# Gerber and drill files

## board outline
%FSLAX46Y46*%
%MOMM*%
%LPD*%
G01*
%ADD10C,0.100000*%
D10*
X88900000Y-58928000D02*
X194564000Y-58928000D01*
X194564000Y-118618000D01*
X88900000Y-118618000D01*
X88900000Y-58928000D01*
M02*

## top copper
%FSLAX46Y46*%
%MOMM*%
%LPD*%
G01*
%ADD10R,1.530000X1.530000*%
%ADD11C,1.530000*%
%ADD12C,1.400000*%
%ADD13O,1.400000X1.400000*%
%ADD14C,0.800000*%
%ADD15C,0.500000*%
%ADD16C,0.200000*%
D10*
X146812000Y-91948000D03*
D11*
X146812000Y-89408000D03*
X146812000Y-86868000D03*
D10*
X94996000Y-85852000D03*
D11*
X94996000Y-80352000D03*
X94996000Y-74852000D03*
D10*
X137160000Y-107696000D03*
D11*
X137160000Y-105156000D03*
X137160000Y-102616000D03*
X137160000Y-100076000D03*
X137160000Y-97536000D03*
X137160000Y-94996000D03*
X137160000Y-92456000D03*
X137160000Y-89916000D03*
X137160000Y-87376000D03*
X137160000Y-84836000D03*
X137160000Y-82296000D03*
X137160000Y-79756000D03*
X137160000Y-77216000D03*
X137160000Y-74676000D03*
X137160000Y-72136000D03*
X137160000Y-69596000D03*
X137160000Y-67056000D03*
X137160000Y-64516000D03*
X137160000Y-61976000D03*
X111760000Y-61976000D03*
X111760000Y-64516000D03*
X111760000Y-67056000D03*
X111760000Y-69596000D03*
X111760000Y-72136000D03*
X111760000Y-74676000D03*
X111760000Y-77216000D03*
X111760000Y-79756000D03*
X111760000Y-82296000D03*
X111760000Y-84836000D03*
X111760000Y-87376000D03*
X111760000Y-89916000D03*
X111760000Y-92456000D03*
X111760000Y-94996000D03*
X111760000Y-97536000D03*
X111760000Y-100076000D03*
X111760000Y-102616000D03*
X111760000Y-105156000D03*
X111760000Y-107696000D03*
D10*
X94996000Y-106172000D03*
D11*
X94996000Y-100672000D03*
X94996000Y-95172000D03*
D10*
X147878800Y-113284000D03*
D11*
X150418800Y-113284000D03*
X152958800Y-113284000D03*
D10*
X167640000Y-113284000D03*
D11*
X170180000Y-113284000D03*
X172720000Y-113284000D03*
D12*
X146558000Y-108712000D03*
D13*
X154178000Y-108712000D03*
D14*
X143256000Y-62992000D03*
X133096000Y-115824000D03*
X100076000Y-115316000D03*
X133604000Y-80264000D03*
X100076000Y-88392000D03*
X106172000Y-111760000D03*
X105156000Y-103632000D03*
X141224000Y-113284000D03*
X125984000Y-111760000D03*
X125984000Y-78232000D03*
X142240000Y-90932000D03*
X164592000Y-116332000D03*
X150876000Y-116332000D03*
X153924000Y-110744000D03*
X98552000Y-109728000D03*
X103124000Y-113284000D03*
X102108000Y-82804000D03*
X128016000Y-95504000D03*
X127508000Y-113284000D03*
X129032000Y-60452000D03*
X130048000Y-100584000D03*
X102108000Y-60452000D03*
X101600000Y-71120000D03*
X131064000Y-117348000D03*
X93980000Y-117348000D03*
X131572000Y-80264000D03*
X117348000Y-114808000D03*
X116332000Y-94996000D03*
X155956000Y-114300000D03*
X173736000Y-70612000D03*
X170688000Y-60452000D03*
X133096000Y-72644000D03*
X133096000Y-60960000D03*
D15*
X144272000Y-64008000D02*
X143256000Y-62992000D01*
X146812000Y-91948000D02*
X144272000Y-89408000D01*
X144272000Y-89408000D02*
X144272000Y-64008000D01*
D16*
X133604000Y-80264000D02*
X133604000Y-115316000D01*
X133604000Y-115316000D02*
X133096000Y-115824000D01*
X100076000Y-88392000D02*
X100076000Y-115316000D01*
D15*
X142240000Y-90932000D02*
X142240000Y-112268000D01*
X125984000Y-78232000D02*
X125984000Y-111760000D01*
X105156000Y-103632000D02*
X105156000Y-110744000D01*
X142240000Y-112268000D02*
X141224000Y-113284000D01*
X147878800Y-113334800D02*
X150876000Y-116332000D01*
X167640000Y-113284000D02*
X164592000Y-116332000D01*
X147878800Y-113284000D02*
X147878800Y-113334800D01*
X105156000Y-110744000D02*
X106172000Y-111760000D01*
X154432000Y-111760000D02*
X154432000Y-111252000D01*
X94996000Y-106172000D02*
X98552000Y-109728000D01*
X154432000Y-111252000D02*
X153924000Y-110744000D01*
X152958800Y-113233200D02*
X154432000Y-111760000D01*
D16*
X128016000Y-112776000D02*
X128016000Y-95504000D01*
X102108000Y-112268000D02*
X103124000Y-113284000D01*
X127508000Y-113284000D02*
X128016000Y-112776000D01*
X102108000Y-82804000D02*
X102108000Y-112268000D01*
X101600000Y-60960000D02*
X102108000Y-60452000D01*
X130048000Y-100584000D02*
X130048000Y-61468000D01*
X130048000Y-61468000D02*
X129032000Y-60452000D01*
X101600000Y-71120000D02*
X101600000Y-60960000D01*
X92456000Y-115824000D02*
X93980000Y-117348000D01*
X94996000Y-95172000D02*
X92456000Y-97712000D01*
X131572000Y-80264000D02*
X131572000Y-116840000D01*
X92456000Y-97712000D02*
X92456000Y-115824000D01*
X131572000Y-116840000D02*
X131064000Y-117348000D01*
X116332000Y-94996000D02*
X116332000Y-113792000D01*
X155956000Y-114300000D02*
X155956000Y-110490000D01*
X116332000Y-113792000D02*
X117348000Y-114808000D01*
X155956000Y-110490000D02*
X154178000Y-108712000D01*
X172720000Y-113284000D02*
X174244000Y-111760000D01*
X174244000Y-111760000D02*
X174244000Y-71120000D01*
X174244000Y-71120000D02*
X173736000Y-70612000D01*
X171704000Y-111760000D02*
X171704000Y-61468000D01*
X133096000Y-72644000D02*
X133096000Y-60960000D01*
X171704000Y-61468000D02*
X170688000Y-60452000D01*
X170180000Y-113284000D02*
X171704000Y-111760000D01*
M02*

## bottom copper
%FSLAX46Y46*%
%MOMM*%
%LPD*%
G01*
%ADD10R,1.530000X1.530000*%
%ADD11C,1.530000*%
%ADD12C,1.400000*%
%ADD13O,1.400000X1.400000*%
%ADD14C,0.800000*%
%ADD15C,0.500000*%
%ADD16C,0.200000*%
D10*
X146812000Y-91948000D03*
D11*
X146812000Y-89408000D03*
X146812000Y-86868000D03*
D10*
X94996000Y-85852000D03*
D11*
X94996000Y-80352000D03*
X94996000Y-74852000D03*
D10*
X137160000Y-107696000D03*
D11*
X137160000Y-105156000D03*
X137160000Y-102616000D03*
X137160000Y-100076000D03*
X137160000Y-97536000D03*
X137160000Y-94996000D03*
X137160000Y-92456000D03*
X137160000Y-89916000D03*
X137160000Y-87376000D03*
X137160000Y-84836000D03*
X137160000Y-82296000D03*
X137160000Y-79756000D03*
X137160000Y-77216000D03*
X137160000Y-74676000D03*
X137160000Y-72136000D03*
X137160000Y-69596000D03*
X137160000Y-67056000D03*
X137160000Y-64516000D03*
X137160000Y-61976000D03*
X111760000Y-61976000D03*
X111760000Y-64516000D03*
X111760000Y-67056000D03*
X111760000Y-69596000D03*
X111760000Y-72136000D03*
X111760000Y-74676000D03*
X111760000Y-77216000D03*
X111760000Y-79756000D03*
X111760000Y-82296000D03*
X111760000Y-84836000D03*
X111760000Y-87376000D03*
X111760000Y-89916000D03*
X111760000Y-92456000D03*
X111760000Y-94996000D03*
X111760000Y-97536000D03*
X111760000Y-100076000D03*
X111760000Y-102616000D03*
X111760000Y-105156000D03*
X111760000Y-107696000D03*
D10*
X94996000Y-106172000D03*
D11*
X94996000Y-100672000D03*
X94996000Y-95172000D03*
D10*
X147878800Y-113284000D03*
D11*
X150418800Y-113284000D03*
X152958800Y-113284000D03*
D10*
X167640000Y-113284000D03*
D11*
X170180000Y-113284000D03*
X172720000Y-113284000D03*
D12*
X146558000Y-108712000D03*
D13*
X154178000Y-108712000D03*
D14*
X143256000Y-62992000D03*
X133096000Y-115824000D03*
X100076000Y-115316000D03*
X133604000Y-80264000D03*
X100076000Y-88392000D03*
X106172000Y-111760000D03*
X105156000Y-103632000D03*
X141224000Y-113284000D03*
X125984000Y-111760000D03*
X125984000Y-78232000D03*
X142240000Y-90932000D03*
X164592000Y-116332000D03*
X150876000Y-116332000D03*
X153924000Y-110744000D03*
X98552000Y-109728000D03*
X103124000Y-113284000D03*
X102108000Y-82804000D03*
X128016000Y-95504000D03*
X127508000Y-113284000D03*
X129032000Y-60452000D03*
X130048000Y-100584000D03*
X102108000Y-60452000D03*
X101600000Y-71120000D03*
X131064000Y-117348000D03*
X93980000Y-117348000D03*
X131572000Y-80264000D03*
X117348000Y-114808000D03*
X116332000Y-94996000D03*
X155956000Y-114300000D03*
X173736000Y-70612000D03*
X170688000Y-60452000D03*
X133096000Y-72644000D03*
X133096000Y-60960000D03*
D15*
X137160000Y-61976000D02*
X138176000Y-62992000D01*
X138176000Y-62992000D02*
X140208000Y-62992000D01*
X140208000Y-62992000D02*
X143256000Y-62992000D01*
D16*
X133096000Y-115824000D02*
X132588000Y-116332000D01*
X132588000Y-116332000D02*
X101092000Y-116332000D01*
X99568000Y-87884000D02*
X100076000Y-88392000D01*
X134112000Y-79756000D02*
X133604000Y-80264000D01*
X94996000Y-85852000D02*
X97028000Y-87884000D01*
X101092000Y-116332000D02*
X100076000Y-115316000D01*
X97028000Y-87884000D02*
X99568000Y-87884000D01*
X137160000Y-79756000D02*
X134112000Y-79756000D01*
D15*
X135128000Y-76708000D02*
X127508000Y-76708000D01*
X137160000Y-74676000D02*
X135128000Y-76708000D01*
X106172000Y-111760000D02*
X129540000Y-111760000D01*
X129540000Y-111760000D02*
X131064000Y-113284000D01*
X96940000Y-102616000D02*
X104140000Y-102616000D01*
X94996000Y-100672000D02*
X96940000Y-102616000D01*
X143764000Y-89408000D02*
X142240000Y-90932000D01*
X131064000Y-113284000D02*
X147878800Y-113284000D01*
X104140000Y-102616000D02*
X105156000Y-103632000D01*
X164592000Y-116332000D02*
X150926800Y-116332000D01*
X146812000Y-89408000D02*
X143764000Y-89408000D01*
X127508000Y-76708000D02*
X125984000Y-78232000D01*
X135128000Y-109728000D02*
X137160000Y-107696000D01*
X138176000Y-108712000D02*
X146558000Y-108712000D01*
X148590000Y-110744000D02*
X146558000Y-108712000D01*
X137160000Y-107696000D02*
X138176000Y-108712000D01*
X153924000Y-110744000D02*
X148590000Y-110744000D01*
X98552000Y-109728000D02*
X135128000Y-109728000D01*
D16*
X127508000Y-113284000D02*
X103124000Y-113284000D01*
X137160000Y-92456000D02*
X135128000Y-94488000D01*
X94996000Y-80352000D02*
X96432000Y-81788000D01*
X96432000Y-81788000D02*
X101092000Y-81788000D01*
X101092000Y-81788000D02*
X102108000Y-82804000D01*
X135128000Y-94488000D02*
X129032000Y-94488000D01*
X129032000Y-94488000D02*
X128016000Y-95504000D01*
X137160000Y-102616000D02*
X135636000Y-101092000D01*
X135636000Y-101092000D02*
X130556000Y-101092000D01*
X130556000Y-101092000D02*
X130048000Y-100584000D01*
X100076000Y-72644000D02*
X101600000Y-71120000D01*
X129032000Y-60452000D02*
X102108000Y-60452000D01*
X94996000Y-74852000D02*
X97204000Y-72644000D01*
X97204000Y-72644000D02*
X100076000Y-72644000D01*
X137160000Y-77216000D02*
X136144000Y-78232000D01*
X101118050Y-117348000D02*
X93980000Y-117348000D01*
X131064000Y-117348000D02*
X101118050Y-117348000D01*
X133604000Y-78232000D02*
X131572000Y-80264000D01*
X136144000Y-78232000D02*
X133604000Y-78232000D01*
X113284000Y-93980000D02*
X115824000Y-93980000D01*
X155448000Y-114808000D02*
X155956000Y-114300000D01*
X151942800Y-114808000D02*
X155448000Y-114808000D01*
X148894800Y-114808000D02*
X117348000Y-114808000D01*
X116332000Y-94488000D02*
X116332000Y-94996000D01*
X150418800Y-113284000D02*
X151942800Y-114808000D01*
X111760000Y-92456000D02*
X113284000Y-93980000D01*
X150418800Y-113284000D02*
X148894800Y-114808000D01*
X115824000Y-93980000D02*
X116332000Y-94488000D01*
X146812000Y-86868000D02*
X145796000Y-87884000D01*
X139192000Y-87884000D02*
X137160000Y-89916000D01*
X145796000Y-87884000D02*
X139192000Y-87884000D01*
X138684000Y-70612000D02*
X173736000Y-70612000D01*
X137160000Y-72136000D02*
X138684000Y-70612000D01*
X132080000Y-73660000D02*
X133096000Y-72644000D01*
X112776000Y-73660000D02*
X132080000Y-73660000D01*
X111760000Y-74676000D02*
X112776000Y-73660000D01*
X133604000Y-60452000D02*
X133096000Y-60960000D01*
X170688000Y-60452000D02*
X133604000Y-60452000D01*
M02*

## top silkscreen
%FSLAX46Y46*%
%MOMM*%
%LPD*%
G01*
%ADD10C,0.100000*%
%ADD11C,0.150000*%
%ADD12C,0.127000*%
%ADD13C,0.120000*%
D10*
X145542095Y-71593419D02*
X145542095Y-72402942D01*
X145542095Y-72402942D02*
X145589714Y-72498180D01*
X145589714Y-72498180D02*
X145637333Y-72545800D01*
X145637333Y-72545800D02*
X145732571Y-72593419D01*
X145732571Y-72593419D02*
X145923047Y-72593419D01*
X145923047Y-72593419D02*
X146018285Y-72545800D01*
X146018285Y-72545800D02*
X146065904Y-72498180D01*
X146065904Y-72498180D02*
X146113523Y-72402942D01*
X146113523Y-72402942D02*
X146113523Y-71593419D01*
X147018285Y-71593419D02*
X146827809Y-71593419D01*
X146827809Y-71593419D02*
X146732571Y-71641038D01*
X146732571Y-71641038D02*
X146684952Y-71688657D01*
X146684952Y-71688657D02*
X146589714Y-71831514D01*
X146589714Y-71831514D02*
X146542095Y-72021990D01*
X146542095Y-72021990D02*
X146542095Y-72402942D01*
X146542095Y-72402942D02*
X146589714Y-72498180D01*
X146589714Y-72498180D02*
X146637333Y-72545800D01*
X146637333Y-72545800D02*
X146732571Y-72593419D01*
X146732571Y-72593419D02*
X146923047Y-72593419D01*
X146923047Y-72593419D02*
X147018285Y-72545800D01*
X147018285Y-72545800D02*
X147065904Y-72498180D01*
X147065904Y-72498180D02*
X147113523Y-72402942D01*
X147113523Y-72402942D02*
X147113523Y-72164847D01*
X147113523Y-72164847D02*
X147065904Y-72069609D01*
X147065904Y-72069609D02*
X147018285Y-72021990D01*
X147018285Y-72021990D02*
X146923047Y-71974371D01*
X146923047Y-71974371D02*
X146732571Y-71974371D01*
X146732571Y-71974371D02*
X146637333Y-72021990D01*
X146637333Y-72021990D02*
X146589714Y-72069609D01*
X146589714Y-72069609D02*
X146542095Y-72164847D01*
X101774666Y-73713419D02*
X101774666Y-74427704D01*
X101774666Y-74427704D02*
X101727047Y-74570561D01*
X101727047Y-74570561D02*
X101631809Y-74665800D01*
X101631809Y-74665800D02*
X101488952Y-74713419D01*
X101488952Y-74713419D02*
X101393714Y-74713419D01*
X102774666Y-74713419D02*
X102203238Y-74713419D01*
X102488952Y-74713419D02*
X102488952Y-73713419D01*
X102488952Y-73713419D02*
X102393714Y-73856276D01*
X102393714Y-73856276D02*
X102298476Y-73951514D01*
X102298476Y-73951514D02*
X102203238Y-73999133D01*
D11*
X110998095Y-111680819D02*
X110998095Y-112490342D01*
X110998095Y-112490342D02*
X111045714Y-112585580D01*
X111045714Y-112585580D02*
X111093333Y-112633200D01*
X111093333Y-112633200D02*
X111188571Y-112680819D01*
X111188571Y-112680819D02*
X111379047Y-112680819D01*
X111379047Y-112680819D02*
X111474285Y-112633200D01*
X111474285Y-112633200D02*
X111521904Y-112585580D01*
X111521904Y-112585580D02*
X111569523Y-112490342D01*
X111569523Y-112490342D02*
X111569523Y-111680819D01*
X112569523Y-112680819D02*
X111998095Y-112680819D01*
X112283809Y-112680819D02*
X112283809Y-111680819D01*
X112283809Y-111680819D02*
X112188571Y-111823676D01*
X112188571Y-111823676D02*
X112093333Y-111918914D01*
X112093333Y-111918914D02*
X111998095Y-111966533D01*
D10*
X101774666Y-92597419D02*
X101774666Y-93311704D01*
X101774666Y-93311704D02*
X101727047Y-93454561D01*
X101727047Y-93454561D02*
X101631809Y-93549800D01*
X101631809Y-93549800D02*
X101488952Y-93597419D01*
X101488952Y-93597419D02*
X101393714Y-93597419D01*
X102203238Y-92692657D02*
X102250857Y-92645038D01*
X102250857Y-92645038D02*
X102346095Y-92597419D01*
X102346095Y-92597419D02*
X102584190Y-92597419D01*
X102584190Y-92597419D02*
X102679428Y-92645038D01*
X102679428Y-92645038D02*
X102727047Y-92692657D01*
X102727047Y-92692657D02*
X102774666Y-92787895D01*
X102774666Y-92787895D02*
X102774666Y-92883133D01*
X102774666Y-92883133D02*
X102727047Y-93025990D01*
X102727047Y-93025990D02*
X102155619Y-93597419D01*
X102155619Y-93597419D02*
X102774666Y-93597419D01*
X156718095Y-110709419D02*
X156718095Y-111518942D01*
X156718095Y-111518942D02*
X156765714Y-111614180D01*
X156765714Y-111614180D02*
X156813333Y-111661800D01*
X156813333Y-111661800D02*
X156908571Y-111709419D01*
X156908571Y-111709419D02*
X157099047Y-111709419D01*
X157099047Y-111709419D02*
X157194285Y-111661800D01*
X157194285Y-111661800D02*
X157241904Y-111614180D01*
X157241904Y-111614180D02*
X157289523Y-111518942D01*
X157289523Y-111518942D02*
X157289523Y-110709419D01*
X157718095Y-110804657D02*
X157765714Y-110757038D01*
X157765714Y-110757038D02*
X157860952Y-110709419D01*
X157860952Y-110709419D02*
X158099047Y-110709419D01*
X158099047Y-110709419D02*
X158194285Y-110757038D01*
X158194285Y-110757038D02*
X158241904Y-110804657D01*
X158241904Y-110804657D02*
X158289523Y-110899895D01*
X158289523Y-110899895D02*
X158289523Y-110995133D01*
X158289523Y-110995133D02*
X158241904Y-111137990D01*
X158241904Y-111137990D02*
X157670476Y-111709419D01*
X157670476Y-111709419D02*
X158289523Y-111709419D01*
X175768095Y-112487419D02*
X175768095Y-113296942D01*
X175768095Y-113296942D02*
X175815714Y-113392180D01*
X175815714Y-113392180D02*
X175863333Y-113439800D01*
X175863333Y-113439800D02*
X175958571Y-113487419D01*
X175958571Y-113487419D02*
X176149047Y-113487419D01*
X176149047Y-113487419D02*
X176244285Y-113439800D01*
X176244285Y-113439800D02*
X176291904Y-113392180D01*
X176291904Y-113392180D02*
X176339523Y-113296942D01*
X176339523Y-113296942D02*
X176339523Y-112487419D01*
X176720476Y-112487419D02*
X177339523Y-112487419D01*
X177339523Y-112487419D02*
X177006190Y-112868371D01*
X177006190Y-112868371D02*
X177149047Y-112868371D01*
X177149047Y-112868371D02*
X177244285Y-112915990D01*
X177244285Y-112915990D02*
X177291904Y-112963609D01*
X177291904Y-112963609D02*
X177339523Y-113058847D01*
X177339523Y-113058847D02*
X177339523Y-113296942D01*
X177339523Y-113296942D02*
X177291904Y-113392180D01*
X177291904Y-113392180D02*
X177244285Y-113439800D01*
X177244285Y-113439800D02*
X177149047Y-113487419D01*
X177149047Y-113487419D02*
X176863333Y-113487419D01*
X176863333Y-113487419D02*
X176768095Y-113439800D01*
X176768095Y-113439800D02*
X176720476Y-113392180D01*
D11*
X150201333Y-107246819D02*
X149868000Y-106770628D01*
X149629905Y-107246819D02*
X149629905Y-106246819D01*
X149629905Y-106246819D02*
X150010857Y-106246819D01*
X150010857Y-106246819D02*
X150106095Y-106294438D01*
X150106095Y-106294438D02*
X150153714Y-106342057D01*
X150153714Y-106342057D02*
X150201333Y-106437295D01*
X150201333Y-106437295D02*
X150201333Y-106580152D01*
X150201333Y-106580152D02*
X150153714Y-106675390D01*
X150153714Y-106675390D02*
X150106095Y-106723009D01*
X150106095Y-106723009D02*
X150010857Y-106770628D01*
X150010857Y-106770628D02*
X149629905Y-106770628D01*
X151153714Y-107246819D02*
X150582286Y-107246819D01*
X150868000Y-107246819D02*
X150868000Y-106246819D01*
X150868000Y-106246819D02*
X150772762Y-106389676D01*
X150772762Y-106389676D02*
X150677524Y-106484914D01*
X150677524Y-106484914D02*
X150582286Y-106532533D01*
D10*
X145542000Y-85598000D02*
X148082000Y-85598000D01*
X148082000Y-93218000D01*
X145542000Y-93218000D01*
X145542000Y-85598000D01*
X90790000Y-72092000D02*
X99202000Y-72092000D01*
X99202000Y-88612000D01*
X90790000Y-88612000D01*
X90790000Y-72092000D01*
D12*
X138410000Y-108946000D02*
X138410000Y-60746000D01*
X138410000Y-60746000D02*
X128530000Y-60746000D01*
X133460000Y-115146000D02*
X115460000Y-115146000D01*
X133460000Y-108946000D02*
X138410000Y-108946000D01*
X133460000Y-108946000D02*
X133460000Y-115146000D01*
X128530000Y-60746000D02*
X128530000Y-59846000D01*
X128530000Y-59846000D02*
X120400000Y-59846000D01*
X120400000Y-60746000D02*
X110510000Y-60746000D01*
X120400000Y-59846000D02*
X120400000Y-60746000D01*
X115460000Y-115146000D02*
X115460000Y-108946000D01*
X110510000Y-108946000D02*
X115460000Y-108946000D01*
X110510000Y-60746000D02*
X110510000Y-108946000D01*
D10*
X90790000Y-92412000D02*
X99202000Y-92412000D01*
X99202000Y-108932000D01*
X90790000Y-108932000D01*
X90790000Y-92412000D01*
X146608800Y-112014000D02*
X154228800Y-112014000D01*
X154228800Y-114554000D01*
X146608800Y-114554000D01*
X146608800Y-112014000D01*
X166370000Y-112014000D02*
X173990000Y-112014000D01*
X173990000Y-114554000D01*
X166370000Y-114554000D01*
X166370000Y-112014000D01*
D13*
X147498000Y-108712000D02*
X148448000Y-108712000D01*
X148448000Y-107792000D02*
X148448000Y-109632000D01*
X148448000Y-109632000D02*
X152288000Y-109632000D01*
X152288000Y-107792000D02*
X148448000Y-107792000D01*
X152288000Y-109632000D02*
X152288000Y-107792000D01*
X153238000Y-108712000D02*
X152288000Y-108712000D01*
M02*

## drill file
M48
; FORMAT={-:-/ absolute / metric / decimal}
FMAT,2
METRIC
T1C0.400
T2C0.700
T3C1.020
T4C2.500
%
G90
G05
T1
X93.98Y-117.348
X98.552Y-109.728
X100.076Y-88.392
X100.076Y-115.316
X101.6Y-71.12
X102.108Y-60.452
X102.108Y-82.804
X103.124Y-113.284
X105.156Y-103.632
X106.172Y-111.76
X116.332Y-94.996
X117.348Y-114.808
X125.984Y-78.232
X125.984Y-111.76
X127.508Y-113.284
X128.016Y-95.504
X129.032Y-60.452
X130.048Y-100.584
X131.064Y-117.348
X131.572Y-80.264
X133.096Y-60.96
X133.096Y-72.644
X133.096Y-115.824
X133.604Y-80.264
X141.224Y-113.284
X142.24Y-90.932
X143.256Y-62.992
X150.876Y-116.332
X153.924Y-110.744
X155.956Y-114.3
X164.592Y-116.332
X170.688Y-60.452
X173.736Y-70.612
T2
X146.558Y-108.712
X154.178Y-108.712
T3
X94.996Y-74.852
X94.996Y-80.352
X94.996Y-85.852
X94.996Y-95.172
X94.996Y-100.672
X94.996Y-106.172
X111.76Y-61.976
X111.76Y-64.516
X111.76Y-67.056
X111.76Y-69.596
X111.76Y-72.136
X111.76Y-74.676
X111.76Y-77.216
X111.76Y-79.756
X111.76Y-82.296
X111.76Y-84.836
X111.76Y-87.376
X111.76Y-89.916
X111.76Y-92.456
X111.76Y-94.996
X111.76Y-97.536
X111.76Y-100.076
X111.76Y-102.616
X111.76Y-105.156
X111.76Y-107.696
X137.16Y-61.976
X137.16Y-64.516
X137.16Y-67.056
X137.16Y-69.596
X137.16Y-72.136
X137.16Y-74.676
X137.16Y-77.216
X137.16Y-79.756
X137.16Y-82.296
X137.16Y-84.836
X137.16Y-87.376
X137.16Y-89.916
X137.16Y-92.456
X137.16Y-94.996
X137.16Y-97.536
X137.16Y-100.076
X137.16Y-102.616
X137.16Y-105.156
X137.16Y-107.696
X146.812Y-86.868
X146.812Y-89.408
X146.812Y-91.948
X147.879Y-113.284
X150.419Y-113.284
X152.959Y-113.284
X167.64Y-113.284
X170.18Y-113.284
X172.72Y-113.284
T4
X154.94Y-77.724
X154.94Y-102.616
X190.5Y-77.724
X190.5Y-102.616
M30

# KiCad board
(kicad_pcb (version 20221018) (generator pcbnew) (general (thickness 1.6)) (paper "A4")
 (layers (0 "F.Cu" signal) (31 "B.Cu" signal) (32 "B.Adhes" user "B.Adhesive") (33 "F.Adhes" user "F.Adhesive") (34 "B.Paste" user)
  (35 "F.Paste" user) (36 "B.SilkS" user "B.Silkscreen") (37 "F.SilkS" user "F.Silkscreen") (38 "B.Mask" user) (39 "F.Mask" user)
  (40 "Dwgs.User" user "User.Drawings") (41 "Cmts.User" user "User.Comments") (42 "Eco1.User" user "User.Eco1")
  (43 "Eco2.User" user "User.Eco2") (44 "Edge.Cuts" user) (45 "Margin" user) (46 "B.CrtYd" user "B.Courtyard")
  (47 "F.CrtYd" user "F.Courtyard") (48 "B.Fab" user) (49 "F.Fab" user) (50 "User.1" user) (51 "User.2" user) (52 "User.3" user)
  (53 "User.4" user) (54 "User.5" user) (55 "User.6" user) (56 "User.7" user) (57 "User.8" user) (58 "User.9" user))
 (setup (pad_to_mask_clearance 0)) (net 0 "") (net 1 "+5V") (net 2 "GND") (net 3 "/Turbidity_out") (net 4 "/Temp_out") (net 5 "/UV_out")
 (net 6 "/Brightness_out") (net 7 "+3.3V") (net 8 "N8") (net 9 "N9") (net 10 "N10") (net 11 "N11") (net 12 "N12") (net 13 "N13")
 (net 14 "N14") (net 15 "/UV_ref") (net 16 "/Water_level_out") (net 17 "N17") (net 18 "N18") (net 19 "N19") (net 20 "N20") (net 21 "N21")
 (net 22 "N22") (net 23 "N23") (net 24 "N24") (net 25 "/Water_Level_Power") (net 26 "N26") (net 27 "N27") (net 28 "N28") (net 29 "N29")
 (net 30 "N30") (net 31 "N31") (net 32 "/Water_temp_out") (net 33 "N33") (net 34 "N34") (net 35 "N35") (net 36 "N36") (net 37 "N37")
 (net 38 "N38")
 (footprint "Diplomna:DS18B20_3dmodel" (layer "F.Cu") (at 149.352 84.328 90)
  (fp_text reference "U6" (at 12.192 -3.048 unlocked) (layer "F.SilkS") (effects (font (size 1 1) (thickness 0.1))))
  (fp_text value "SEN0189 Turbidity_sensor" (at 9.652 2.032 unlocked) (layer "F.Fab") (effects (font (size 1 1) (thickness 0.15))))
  (fp_rect (start -8.89 -3.81) (end -1.27 -1.27) (stroke (width 0.1) (type default)) (fill none) (layer "F.SilkS"))
  (pad "1" thru_hole rect (at -7.62 -2.54 90) (size 1.53 1.53) (drill 1.02) (layers "*.Cu" "*.Mask") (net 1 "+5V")
   (solder_mask_margin 0.102))
  (pad "2" thru_hole circle (at -5.08 -2.54 90) (size 1.53 1.53) (drill 1.02) (layers "*.Cu" "*.Mask") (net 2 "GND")
   (solder_mask_margin 0.102))
  (pad "3" thru_hole circle (at -2.54 -2.54 90) (size 1.53 1.53) (drill 1.02) (layers "*.Cu" "*.Mask") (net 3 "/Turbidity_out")
   (solder_mask_margin 0.102)))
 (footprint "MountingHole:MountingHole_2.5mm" (layer "F.Cu") (at 190.5 102.616)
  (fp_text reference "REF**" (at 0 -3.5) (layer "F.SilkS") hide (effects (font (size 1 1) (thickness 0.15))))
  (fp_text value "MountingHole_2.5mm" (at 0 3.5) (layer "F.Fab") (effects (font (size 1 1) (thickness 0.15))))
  (pad "" np_thru_hole circle (at 0 0) (size 2.5 2.5) (drill 2.5) (layers "F&B.Cu" "*.Mask")))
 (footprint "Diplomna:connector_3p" (layer "F.Cu") (at 94.996 80.352 90)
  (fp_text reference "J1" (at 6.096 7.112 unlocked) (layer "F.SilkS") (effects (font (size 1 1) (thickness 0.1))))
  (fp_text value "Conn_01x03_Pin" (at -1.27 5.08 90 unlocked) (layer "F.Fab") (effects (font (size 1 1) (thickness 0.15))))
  (fp_rect (start -8.26 -4.206) (end 8.26 4.206) (stroke (width 0.1) (type default)) (fill none) (layer "F.SilkS"))
  (pad "1" thru_hole rect (at -5.5 0 90) (size 1.53 1.53) (drill 1.02) (layers "*.Cu" "*.Mask") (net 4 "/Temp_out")
   (solder_mask_margin 0.102))
  (pad "2" thru_hole circle (at 0 0 90) (size 1.53 1.53) (drill 1.02) (layers "*.Cu" "*.Mask") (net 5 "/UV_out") (solder_mask_margin 0.102))
  (pad "3" thru_hole circle (at 5.5 0 90) (size 1.53 1.53) (drill 1.02) (layers "*.Cu" "*.Mask") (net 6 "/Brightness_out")
   (solder_mask_margin 0.102)))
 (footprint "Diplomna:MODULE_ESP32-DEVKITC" (layer "F.Cu") (at 124.46 84.846 180)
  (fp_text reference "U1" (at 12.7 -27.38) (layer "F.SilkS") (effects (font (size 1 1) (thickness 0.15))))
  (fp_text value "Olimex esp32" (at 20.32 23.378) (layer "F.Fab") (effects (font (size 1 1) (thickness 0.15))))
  (fp_line (start -13.95 -24.1) (end -13.95 24.1) (stroke (width 0.127) (type solid)) (layer "F.SilkS"))
  (fp_line (start -13.95 24.1) (end -4.07 24.1) (stroke (width 0.127) (type solid)) (layer "F.SilkS"))
  (fp_line (start -9 -30.3) (end 9 -30.3) (stroke (width 0.127) (type solid)) (layer "F.SilkS"))
  (fp_line (start -9 -24.1) (end -13.95 -24.1) (stroke (width 0.127) (type solid)) (layer "F.SilkS"))
  (fp_line (start -9 -24.1) (end -9 -30.3) (stroke (width 0.127) (type solid)) (layer "F.SilkS"))
  (fp_line (start -4.07 24.1) (end -4.07 25) (stroke (width 0.127) (type solid)) (layer "F.SilkS"))
  (fp_line (start -4.07 25) (end 4.06 25) (stroke (width 0.127) (type solid)) (layer "F.SilkS"))
  (fp_line (start 4.06 24.1) (end 13.95 24.1) (stroke (width 0.127) (type solid)) (layer "F.SilkS"))
  (fp_line (start 4.06 25) (end 4.06 24.1) (stroke (width 0.127) (type solid)) (layer "F.SilkS"))
  (fp_line (start 9 -30.3) (end 9 -24.1) (stroke (width 0.127) (type solid)) (layer "F.SilkS"))
  (fp_line (start 13.95 -24.1) (end 9 -24.1) (stroke (width 0.127) (type solid)) (layer "F.SilkS"))
  (fp_line (start 13.95 24.1) (end 13.95 -24.1) (stroke (width 0.127) (type solid)) (layer "F.SilkS"))
  (pad "1" thru_hole rect (at -12.7 -22.85 180) (size 1.53 1.53) (drill 1.02) (layers "*.Cu" "*.Mask") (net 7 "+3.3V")
   (solder_mask_margin 0.102))
  (pad "2" thru_hole circle (at -12.7 -20.31 180) (size 1.53 1.53) (drill 1.02) (layers "*.Cu" "*.Mask") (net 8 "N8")
   (solder_mask_margin 0.102))
  (pad "3" thru_hole circle (at -12.7 -17.77 180) (size 1.53 1.53) (drill 1.02) (layers "*.Cu" "*.Mask") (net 6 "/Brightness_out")
   (solder_mask_margin 0.102))
  (pad "4" thru_hole circle (at -12.7 -15.23 180) (size 1.53 1.53) (drill 1.02) (layers "*.Cu" "*.Mask") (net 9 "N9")
   (solder_mask_margin 0.102))
  (pad "5" thru_hole circle (at -12.7 -12.69 180) (size 1.53 1.53) (drill 1.02) (layers "*.Cu" "*.Mask") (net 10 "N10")
   (solder_mask_margin 0.102))
  (pad "6" thru_hole circle (at -12.7 -10.15 180) (size 1.53 1.53) (drill 1.02) (layers "*.Cu" "*.Mask") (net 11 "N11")
   (solder_mask_margin 0.102))
  (pad "7" thru_hole circle (at -12.7 -7.61 180) (size 1.53 1.53) (drill 1.02) (layers "*.Cu" "*.Mask") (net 5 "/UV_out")
   (solder_mask_margin 0.102))
  (pad "8" thru_hole circle (at -12.7 -5.07 180) (size 1.53 1.53) (drill 1.02) (layers "*.Cu" "*.Mask") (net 3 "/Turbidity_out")
   (solder_mask_margin 0.102))
  (pad "9" thru_hole circle (at -12.7 -2.53 180) (size 1.53 1.53) (drill 1.02) (layers "*.Cu" "*.Mask") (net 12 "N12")
   (solder_mask_margin 0.102))
  (pad "10" thru_hole circle (at -12.7 0.01 180) (size 1.53 1.53) (drill 1.02) (layers "*.Cu" "*.Mask") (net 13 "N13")
   (solder_mask_margin 0.102))
  (pad "11" thru_hole circle (at -12.7 2.55 180) (size 1.53 1.53) (drill 1.02) (layers "*.Cu" "*.Mask") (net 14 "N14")
   (solder_mask_margin 0.102))
  (pad "12" thru_hole circle (at -12.7 5.09 180) (size 1.53 1.53) (drill 1.02) (layers "*.Cu" "*.Mask") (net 4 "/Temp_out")
   (solder_mask_margin 0.102))
  (pad "13" thru_hole circle (at -12.7 7.63 180) (size 1.53 1.53) (drill 1.02) (layers "*.Cu" "*.Mask") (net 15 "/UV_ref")
   (solder_mask_margin 0.102))
  (pad "14" thru_hole circle (at -12.7 10.17 180) (size 1.53 1.53) (drill 1.02) (layers "*.Cu" "*.Mask") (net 2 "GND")
   (solder_mask_margin 0.102))
  (pad "15" thru_hole circle (at -12.7 12.71 180) (size 1.53 1.53) (drill 1.02) (layers "*.Cu" "*.Mask") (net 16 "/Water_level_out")
   (solder_mask_margin 0.102))
  (pad "16" thru_hole circle (at -12.7 15.25 180) (size 1.53 1.53) (drill 1.02) (layers "*.Cu" "*.Mask") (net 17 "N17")
   (solder_mask_margin 0.102))
  (pad "17" thru_hole circle (at -12.7 17.79 180) (size 1.53 1.53) (drill 1.02) (layers "*.Cu" "*.Mask") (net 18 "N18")
   (solder_mask_margin 0.102))
  (pad "18" thru_hole circle (at -12.7 20.33 180) (size 1.53 1.53) (drill 1.02) (layers "*.Cu" "*.Mask") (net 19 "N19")
   (solder_mask_margin 0.102))
  (pad "19" thru_hole circle (at -12.7 22.87 180) (size 1.53 1.53) (drill 1.02) (layers "*.Cu" "*.Mask") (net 1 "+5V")
   (solder_mask_margin 0.102))
  (pad "20" thru_hole circle (at 12.7 22.87 180) (size 1.53 1.53) (drill 1.02) (layers "*.Cu" "*.Mask") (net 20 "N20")
   (solder_mask_margin 0.102))
  (pad "21" thru_hole circle (at 12.7 20.33 180) (size 1.53 1.53) (drill 1.02) (layers "*.Cu" "*.Mask") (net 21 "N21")
   (solder_mask_margin 0.102))
  (pad "22" thru_hole circle (at 12.7 17.79 180) (size 1.53 1.53) (drill 1.02) (layers "*.Cu" "*.Mask") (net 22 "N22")
   (solder_mask_margin 0.102))
  (pad "23" thru_hole circle (at 12.7 15.25 180) (size 1.53 1.53) (drill 1.02) (layers "*.Cu" "*.Mask") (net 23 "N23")
   (solder_mask_margin 0.102))
  (pad "24" thru_hole circle (at 12.7 12.71 180) (size 1.53 1.53) (drill 1.02) (layers "*.Cu" "*.Mask") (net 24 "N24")
   (solder_mask_margin 0.102))
  (pad "25" thru_hole circle (at 12.7 10.17 180) (size 1.53 1.53) (drill 1.02) (layers "*.Cu" "*.Mask") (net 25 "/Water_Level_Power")
   (solder_mask_margin 0.102))
  (pad "26" thru_hole circle (at 12.7 7.63 180) (size 1.53 1.53) (drill 1.02) (layers "*.Cu" "*.Mask") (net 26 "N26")
   (solder_mask_margin 0.102))
  (pad "27" thru_hole circle (at 12.7 5.09 180) (size 1.53 1.53) (drill 1.02) (layers "*.Cu" "*.Mask") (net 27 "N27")
   (solder_mask_margin 0.102))
  (pad "28" thru_hole circle (at 12.7 2.55 180) (size 1.53 1.53) (drill 1.02) (layers "*.Cu" "*.Mask") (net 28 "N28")
   (solder_mask_margin 0.102))
  (pad "29" thru_hole circle (at 12.7 0.01 180) (size 1.53 1.53) (drill 1.02) (layers "*.Cu" "*.Mask") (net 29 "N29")
   (solder_mask_margin 0.102))
  (pad "30" thru_hole circle (at 12.7 -2.53 180) (size 1.53 1.53) (drill 1.02) (layers "*.Cu" "*.Mask") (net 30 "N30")
   (solder_mask_margin 0.102))
  (pad "31" thru_hole circle (at 12.7 -5.07 180) (size 1.53 1.53) (drill 1.02) (layers "*.Cu" "*.Mask") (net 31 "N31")
   (solder_mask_margin 0.102))
  (pad "32" thru_hole circle (at 12.7 -7.61 180) (size 1.53 1.53) (drill 1.02) (layers "*.Cu" "*.Mask") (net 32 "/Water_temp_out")
   (solder_mask_margin 0.102))
  (pad "33" thru_hole circle (at 12.7 -10.15 180) (size 1.53 1.53) (drill 1.02) (layers "*.Cu" "*.Mask") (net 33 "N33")
   (solder_mask_margin 0.102))
  (pad "34" thru_hole circle (at 12.7 -12.69 180) (size 1.53 1.53) (drill 1.02) (layers "*.Cu" "*.Mask") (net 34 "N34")
   (solder_mask_margin 0.102))
  (pad "35" thru_hole circle (at 12.7 -15.23 180) (size 1.53 1.53) (drill 1.02) (layers "*.Cu" "*.Mask") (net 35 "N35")
   (solder_mask_margin 0.102))
  (pad "36" thru_hole circle (at 12.7 -17.77 180) (size 1.53 1.53) (drill 1.02) (layers "*.Cu" "*.Mask") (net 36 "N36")
   (solder_mask_margin 0.102))
  (pad "37" thru_hole circle (at 12.7 -20.31 180) (size 1.53 1.53) (drill 1.02) (layers "*.Cu" "*.Mask") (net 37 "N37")
   (solder_mask_margin 0.102))
  (pad "38" thru_hole circle (at 12.7 -22.85 180) (size 1.53 1.53) (drill 1.02) (layers "*.Cu" "*.Mask") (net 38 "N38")
   (solder_mask_margin 0.102)))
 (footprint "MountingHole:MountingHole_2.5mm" (layer "F.Cu") (at 190.5 77.724)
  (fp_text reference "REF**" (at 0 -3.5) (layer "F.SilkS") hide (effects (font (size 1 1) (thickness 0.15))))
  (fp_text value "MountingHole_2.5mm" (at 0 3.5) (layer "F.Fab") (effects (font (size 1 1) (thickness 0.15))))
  (pad "" np_thru_hole circle (at 0 0) (size 2.5 2.5) (drill 2.5) (layers "F&B.Cu" "*.Mask")))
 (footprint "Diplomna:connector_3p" (layer "F.Cu") (at 94.996 100.672 90)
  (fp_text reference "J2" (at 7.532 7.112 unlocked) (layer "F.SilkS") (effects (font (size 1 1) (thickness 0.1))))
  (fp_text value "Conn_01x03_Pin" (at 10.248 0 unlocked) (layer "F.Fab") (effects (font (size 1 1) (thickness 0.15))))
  (fp_rect (start -8.26 -4.206) (end 8.26 4.206) (stroke (width 0.1) (type default)) (fill none) (layer "F.SilkS"))
  (pad "1" thru_hole rect (at -5.5 0 90) (size 1.53 1.53) (drill 1.02) (layers "*.Cu" "*.Mask") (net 7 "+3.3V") (solder_mask_margin 0.102))
  (pad "2" thru_hole circle (at 0 0 90) (size 1.53 1.53) (drill 1.02) (layers "*.Cu" "*.Mask") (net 2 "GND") (solder_mask_margin 0.102))
  (pad "3" thru_hole circle (at 5.5 0 90) (size 1.53 1.53) (drill 1.02) (layers "*.Cu" "*.Mask") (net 15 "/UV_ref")
   (solder_mask_margin 0.102)))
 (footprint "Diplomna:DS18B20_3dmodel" (layer "F.Cu") (at 155.4988 115.824)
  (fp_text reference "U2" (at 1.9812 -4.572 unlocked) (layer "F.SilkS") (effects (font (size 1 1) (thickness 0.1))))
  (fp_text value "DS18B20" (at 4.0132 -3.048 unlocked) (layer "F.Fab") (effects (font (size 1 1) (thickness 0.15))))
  (fp_rect (start -8.89 -3.81) (end -1.27 -1.27) (stroke (width 0.1) (type default)) (fill none) (layer "F.SilkS"))
  (pad "1" thru_hole rect (at -7.62 -2.54) (size 1.53 1.53) (drill 1.02) (layers "*.Cu" "*.Mask") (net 2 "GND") (solder_mask_margin 0.102))
  (pad "2" thru_hole circle (at -5.08 -2.54) (size 1.53 1.53) (drill 1.02) (layers "*.Cu" "*.Mask") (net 32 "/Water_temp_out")
   (solder_mask_margin 0.102))
  (pad "3" thru_hole circle (at -2.54 -2.54) (size 1.53 1.53) (drill 1.02) (layers "*.Cu" "*.Mask") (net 7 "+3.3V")
   (solder_mask_margin 0.102)))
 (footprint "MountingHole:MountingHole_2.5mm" (layer "F.Cu") (at 154.94 102.616)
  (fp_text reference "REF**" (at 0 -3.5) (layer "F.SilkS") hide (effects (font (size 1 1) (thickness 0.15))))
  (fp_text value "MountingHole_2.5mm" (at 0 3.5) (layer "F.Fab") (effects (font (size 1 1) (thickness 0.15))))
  (pad "" np_thru_hole circle (at 0 0) (size 2.5 2.5) (drill 2.5) (layers "*.Cu" "*.Mask")))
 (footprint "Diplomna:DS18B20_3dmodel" (layer "F.Cu") (at 175.26 115.824)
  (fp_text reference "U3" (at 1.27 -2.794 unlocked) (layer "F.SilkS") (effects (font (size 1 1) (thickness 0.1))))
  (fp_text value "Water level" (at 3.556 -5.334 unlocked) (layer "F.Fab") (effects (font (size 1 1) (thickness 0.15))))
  (fp_rect (start -8.89 -3.81) (end -1.27 -1.27) (stroke (width 0.1) (type default)) (fill none) (layer "F.SilkS"))
  (pad "1" thru_hole rect (at -7.62 -2.54) (size 1.53 1.53) (drill 1.02) (layers "*.Cu" "*.Mask") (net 2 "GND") (solder_mask_margin 0.102))
  (pad "2" thru_hole circle (at -5.08 -2.54) (size 1.53 1.53) (drill 1.02) (layers "*.Cu" "*.Mask") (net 25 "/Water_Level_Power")
   (solder_mask_margin 0.102))
  (pad "3" thru_hole circle (at -2.54 -2.54) (size 1.53 1.53) (drill 1.02) (layers "*.Cu" "*.Mask") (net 16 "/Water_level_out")
   (solder_mask_margin 0.102)))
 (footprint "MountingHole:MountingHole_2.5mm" (layer "F.Cu") (at 154.94 77.724)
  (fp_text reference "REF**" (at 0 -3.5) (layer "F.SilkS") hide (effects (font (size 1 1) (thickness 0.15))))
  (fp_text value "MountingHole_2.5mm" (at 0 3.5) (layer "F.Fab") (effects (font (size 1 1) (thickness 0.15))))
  (pad "" np_thru_hole circle (at 0 0) (size 2.5 2.5) (drill 2.5) (layers "F&B.Cu" "*.Mask")))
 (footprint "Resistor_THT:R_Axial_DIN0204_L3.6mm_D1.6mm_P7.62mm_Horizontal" (layer "F.Cu") (at 146.558 108.712)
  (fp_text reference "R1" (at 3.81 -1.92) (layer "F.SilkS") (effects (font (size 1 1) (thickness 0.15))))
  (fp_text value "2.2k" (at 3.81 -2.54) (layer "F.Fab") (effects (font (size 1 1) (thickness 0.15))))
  (fp_line (start 0.94 0) (end 1.89 0) (stroke (width 0.12) (type solid)) (layer "F.SilkS"))
  (fp_line (start 1.89 -0.92) (end 1.89 0.92) (stroke (width 0.12) (type solid)) (layer "F.SilkS"))
  (fp_line (start 1.89 0.92) (end 5.73 0.92) (stroke (width 0.12) (type solid)) (layer "F.SilkS"))
  (fp_line (start 5.73 -0.92) (end 1.89 -0.92) (stroke (width 0.12) (type solid)) (layer "F.SilkS"))
  (fp_line (start 5.73 0.92) (end 5.73 -0.92) (stroke (width 0.12) (type solid)) (layer "F.SilkS"))
  (fp_line (start 6.68 0) (end 5.73 0) (stroke (width 0.12) (type solid)) (layer "F.SilkS"))
  (pad "1" thru_hole circle (at 0 0) (size 1.4 1.4) (drill 0.7) (layers "*.Cu" "*.Mask") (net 7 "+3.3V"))
  (pad "2" thru_hole oval (at 7.62 0) (size 1.4 1.4) (drill 0.7) (layers "*.Cu" "*.Mask") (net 32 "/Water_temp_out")))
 (gr_rect (start 88.9 58.928) (end 194.564 118.618) (stroke (width 0.1) (type default)) (fill none) (layer "Edge.Cuts"))
 (segment (start 144.272 64.008) (end 143.256 62.992) (width 0.5) (layer "F.Cu") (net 1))
 (segment (start 146.812 91.948) (end 144.272 89.408) (width 0.5) (layer "F.Cu") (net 1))
 (segment (start 144.272 89.408) (end 144.272 64.008) (width 0.5) (layer "F.Cu") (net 1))
 (via (at 143.256 62.992) (size 0.8) (drill 0.4) (layers "F.Cu" "B.Cu") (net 1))
 (segment (start 137.16 61.976) (end 138.176 62.992) (width 0.5) (layer "B.Cu") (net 1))
 (segment (start 138.176 62.992) (end 140.208 62.992) (width 0.5) (layer "B.Cu") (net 1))
 (segment (start 140.208 62.992) (end 143.256 62.992) (width 0.5) (layer "B.Cu") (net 1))
 (segment (start 133.604 80.264) (end 133.604 115.316) (width 0.2) (layer "F.Cu") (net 4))
 (segment (start 133.604 115.316) (end 133.096 115.824) (width 0.2) (layer "F.Cu") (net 4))
 (segment (start 100.076 88.392) (end 100.076 115.316) (width 0.2) (layer "F.Cu") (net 4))
 (via (at 133.096 115.824) (size 0.8) (drill 0.4) (layers "F.Cu" "B.Cu") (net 4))
 (via (at 100.076 115.316) (size 0.8) (drill 0.4) (layers "F.Cu" "B.Cu") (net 4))
 (via (at 133.604 80.264) (size 0.8) (drill 0.4) (layers "F.Cu" "B.Cu") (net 4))
 (via (at 100.076 88.392) (size 0.8) (drill 0.4) (layers "F.Cu" "B.Cu") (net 4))
 (segment (start 133.096 115.824) (end 132.588 116.332) (width 0.2) (layer "B.Cu") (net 4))
 (segment (start 132.588 116.332) (end 101.092 116.332) (width 0.2) (layer "B.Cu") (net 4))
 (segment (start 99.568 87.884) (end 100.076 88.392) (width 0.2) (layer "B.Cu") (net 4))
 (segment (start 134.112 79.756) (end 133.604 80.264) (width 0.2) (layer "B.Cu") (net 4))
 (segment (start 94.996 85.852) (end 97.028 87.884) (width 0.2) (layer "B.Cu") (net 4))
 (segment (start 101.092 116.332) (end 100.076 115.316) (width 0.2) (layer "B.Cu") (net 4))
 (segment (start 97.028 87.884) (end 99.568 87.884) (width 0.2) (layer "B.Cu") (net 4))
 (segment (start 137.16 79.756) (end 134.112 79.756) (width 0.2) (layer "B.Cu") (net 4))
 (segment (start 142.24 90.932) (end 142.24 112.268) (width 0.5) (layer "F.Cu") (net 2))
 (segment (start 125.984 78.232) (end 125.984 111.76) (width 0.5) (layer "F.Cu") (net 2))
 (segment (start 105.156 103.632) (end 105.156 110.744) (width 0.5) (layer "F.Cu") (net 2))
 (segment (start 142.24 112.268) (end 141.224 113.284) (width 0.5) (layer "F.Cu") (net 2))
 (segment (start 147.8788 113.3348) (end 150.876 116.332) (width 0.5) (layer "F.Cu") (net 2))
 (segment (start 167.64 113.284) (end 164.592 116.332) (width 0.5) (layer "F.Cu") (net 2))
 (segment (start 147.8788 113.284) (end 147.8788 113.3348) (width 0.5) (layer "F.Cu") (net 2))
 (segment (start 105.156 110.744) (end 106.172 111.76) (width 0.5) (layer "F.Cu") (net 2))
 (via (at 106.172 111.76) (size 0.8) (drill 0.4) (layers "F.Cu" "B.Cu") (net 2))
 (via (at 105.156 103.632) (size 0.8) (drill 0.4) (layers "F.Cu" "B.Cu") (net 2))
 (via (at 141.224 113.284) (size 0.8) (drill 0.4) (layers "F.Cu" "B.Cu") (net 2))
 (via (at 125.984 111.76) (size 0.8) (drill 0.4) (layers "F.Cu" "B.Cu") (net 2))
 (via (at 125.984 78.232) (size 0.8) (drill 0.4) (layers "F.Cu" "B.Cu") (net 2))
 (via (at 142.24 90.932) (size 0.8) (drill 0.4) (layers "F.Cu" "B.Cu") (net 2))
 (via (at 164.592 116.332) (size 0.8) (drill 0.4) (layers "F.Cu" "B.Cu") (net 2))
 (via (at 150.876 116.332) (size 0.8) (drill 0.4) (layers "F.Cu" "B.Cu") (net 2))
 (segment (start 135.128 76.708) (end 127.508 76.708) (width 0.5) (layer "B.Cu") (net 2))
 (segment (start 137.16 74.676) (end 135.128 76.708) (width 0.5) (layer "B.Cu") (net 2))
 (segment (start 106.172 111.76) (end 129.54 111.76) (width 0.5) (layer "B.Cu") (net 2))
 (segment (start 129.54 111.76) (end 131.064 113.284) (width 0.5) (layer "B.Cu") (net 2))
 (segment (start 96.94 102.616) (end 104.14 102.616) (width 0.5) (layer "B.Cu") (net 2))
 (segment (start 94.996 100.672) (end 96.94 102.616) (width 0.5) (layer "B.Cu") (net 2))
 (segment (start 143.764 89.408) (end 142.24 90.932) (width 0.5) (layer "B.Cu") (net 2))
 (segment (start 131.064 113.284) (end 147.8788 113.284) (width 0.5) (layer "B.Cu") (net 2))
 (segment (start 104.14 102.616) (end 105.156 103.632) (width 0.5) (layer "B.Cu") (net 2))
 (segment (start 164.592 116.332) (end 150.9268 116.332) (width 0.5) (layer "B.Cu") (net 2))
 (segment (start 146.812 89.408) (end 143.764 89.408) (width 0.5) (layer "B.Cu") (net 2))
 (segment (start 127.508 76.708) (end 125.984 78.232) (width 0.5) (layer "B.Cu") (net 2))
 (segment (start 154.432 111.76) (end 154.432 111.252) (width 0.5) (layer "F.Cu") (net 7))
 (segment (start 94.996 106.172) (end 98.552 109.728) (width 0.5) (layer "F.Cu") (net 7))
 (segment (start 154.432 111.252) (end 153.924 110.744) (width 0.5) (layer "F.Cu") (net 7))
 (segment (start 152.9588 113.2332) (end 154.432 111.76) (width 0.5) (layer "F.Cu") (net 7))
 (via (at 153.924 110.744) (size 0.8) (drill 0.4) (layers "F.Cu" "B.Cu") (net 7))
 (via (at 98.552 109.728) (size 0.8) (drill 0.4) (layers "F.Cu" "B.Cu") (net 7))
 (segment (start 135.128 109.728) (end 137.16 107.696) (width 0.5) (layer "B.Cu") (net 7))
 (segment (start 138.176 108.712) (end 146.558 108.712) (width 0.5) (layer "B.Cu") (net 7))
 (segment (start 148.59 110.744) (end 146.558 108.712) (width 0.5) (layer "B.Cu") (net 7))
 (segment (start 137.16 107.696) (end 138.176 108.712) (width 0.5) (layer "B.Cu") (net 7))
 (segment (start 153.924 110.744) (end 148.59 110.744) (width 0.5) (layer "B.Cu") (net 7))
 (segment (start 98.552 109.728) (end 135.128 109.728) (width 0.5) (layer "B.Cu") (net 7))
 (segment (start 128.016 112.776) (end 128.016 95.504) (width 0.2) (layer "F.Cu") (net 5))
 (segment (start 102.108 112.268) (end 103.124 113.284) (width 0.2) (layer "F.Cu") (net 5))
 (segment (start 127.508 113.284) (end 128.016 112.776) (width 0.2) (layer "F.Cu") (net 5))
 (segment (start 102.108 82.804) (end 102.108 112.268) (width 0.2) (layer "F.Cu") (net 5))
 (via (at 103.124 113.284) (size 0.8) (drill 0.4) (layers "F.Cu" "B.Cu") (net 5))
 (via (at 102.108 82.804) (size 0.8) (drill 0.4) (layers "F.Cu" "B.Cu") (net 5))
 (via (at 128.016 95.504) (size 0.8) (drill 0.4) (layers "F.Cu" "B.Cu") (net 5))
 (via (at 127.508 113.284) (size 0.8) (drill 0.4) (layers "F.Cu" "B.Cu") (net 5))
 (segment (start 127.508 113.284) (end 103.124 113.284) (width 0.2) (layer "B.Cu") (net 5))
 (segment (start 137.16 92.456) (end 135.128 94.488) (width 0.2) (layer "B.Cu") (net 5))
 (segment (start 94.996 80.352) (end 96.432 81.788) (width 0.2) (layer "B.Cu") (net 5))
 (segment (start 96.432 81.788) (end 101.092 81.788) (width 0.2) (layer "B.Cu") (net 5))
 (segment (start 101.092 81.788) (end 102.108 82.804) (width 0.2) (layer "B.Cu") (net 5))
 (segment (start 135.128 94.488) (end 129.032 94.488) (width 0.2) (layer "B.Cu") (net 5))
 (segment (start 129.032 94.488) (end 128.016 95.504) (width 0.2) (layer "B.Cu") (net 5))
 (segment (start 101.6 60.96) (end 102.108 60.452) (width 0.2) (layer "F.Cu") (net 6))
 (segment (start 130.048 100.584) (end 130.048 61.468) (width 0.2) (layer "F.Cu") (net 6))
 (segment (start 130.048 61.468) (end 129.032 60.452) (width 0.2) (layer "F.Cu") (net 6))
 (segment (start 101.6 71.12) (end 101.6 60.96) (width 0.2) (layer "F.Cu") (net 6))
 (via (at 129.032 60.452) (size 0.8) (drill 0.4) (layers "F.Cu" "B.Cu") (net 6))
 (via (at 130.048 100.584) (size 0.8) (drill 0.4) (layers "F.Cu" "B.Cu") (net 6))
 (via (at 102.108 60.452) (size 0.8) (drill 0.4) (layers "F.Cu" "B.Cu") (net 6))
 (via (at 101.6 71.12) (size 0.8) (drill 0.4) (layers "F.Cu" "B.Cu") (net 6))
 (segment (start 137.16 102.616) (end 135.636 101.092) (width 0.2) (layer "B.Cu") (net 6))
 (segment (start 135.636 101.092) (end 130.556 101.092) (width 0.2) (layer "B.Cu") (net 6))
 (segment (start 130.556 101.092) (end 130.048 100.584) (width 0.2) (layer "B.Cu") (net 6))
 (segment (start 100.076 72.644) (end 101.6 71.12) (width 0.2) (layer "B.Cu") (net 6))
 (segment (start 129.032 60.452) (end 102.108 60.452) (width 0.2) (layer "B.Cu") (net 6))
 (segment (start 94.996 74.852) (end 97.204 72.644) (width 0.2) (layer "B.Cu") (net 6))
 (segment (start 97.204 72.644) (end 100.076 72.644) (width 0.2) (layer "B.Cu") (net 6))
 (segment (start 92.456 115.824) (end 93.98 117.348) (width 0.2) (layer "F.Cu") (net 15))
 (segment (start 94.996 95.172) (end 92.456 97.712) (width 0.2) (layer "F.Cu") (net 15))
 (segment (start 131.572 80.264) (end 131.572 116.84) (width 0.2) (layer "F.Cu") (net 15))
 (segment (start 92.456 97.712) (end 92.456 115.824) (width 0.2) (layer "F.Cu") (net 15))
 (segment (start 131.572 116.84) (end 131.064 117.348) (width 0.2) (layer "F.Cu") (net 15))
 (via (at 131.064 117.348) (size 0.8) (drill 0.4) (layers "F.Cu" "B.Cu") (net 15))
 (via (at 93.98 117.348) (size 0.8) (drill 0.4) (layers "F.Cu" "B.Cu") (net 15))
 (via (at 131.572 80.264) (size 0.8) (drill 0.4) (layers "F.Cu" "B.Cu") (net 15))
 (segment (start 137.16 77.216) (end 136.144 78.232) (width 0.2) (layer "B.Cu") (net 15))
 (segment (start 101.11805 117.348) (end 93.98 117.348) (width 0.2) (layer "B.Cu") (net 15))
 (segment (start 131.064 117.348) (end 101.11805 117.348) (width 0.2) (layer "B.Cu") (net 15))
 (segment (start 133.604 78.232) (end 131.572 80.264) (width 0.2) (layer "B.Cu") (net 15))
 (segment (start 136.144 78.232) (end 133.604 78.232) (width 0.2) (layer "B.Cu") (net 15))
 (segment (start 116.332 94.996) (end 116.332 113.792) (width 0.2) (layer "F.Cu") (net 32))
 (segment (start 155.956 114.3) (end 155.956 110.49) (width 0.2) (layer "F.Cu") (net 32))
 (segment (start 116.332 113.792) (end 117.348 114.808) (width 0.2) (layer "F.Cu") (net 32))
 (segment (start 155.956 110.49) (end 154.178 108.712) (width 0.2) (layer "F.Cu") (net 32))
 (via (at 117.348 114.808) (size 0.8) (drill 0.4) (layers "F.Cu" "B.Cu") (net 32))
 (via (at 116.332 94.996) (size 0.8) (drill 0.4) (layers "F.Cu" "B.Cu") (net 32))
 (via (at 155.956 114.3) (size 0.8) (drill 0.4) (layers "F.Cu" "B.Cu") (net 32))
 (segment (start 113.284 93.98) (end 115.824 93.98) (width 0.2) (layer "B.Cu") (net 32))
 (segment (start 155.448 114.808) (end 155.956 114.3) (width 0.2) (layer "B.Cu") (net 32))
 (segment (start 151.9428 114.808) (end 155.448 114.808) (width 0.2) (layer "B.Cu") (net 32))
 (segment (start 148.8948 114.808) (end 117.348 114.808) (width 0.2) (layer "B.Cu") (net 32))
 (segment (start 116.332 94.488) (end 116.332 94.996) (width 0.2) (layer "B.Cu") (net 32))
 (segment (start 150.4188 113.284) (end 151.9428 114.808) (width 0.2) (layer "B.Cu") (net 32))
 (segment (start 111.76 92.456) (end 113.284 93.98) (width 0.2) (layer "B.Cu") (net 32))
 (segment (start 150.4188 113.284) (end 148.8948 114.808) (width 0.2) (layer "B.Cu") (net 32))
 (segment (start 115.824 93.98) (end 116.332 94.488) (width 0.2) (layer "B.Cu") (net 32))
 (segment (start 146.812 86.868) (end 145.796 87.884) (width 0.2) (layer "B.Cu") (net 3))
 (segment (start 139.192 87.884) (end 137.16 89.916) (width 0.2) (layer "B.Cu") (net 3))
 (segment (start 145.796 87.884) (end 139.192 87.884) (width 0.2) (layer "B.Cu") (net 3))
 (segment (start 172.72 113.284) (end 174.244 111.76) (width 0.2) (layer "F.Cu") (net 16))
 (segment (start 174.244 111.76) (end 174.244 71.12) (width 0.2) (layer "F.Cu") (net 16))
 (segment (start 174.244 71.12) (end 173.736 70.612) (width 0.2) (layer "F.Cu") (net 16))
 (via (at 173.736 70.612) (size 0.8) (drill 0.4) (layers "F.Cu" "B.Cu") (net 16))
 (segment (start 138.684 70.612) (end 173.736 70.612) (width 0.2) (layer "B.Cu") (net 16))
 (segment (start 137.16 72.136) (end 138.684 70.612) (width 0.2) (layer "B.Cu") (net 16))
 (segment (start 171.704 111.76) (end 171.704 61.468) (width 0.2) (layer "F.Cu") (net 25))
 (segment (start 133.096 72.644) (end 133.096 60.96) (width 0.2) (layer "F.Cu") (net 25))
 (segment (start 171.704 61.468) (end 170.688 60.452) (width 0.2) (layer "F.Cu") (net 25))
 (segment (start 170.18 113.284) (end 171.704 111.76) (width 0.2) (layer "F.Cu") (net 25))
 (via (at 170.688 60.452) (size 0.8) (drill 0.4) (layers "F.Cu" "B.Cu") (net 25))
 (via (at 133.096 72.644) (size 0.8) (drill 0.4) (layers "F.Cu" "B.Cu") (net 25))
 (via (at 133.096 60.96) (size 0.8) (drill 0.4) (layers "F.Cu" "B.Cu") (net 25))
 (segment (start 132.08 73.66) (end 133.096 72.644) (width 0.2) (layer "B.Cu") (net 25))
 (segment (start 112.776 73.66) (end 132.08 73.66) (width 0.2) (layer "B.Cu") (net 25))
 (segment (start 111.76 74.676) (end 112.776 73.66) (width 0.2) (layer "B.Cu") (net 25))
 (segment (start 133.604 60.452) (end 133.096 60.96) (width 0.2) (layer "B.Cu") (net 25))
 (segment (start 170.688 60.452) (end 133.604 60.452) (width 0.2) (layer "B.Cu") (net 25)))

